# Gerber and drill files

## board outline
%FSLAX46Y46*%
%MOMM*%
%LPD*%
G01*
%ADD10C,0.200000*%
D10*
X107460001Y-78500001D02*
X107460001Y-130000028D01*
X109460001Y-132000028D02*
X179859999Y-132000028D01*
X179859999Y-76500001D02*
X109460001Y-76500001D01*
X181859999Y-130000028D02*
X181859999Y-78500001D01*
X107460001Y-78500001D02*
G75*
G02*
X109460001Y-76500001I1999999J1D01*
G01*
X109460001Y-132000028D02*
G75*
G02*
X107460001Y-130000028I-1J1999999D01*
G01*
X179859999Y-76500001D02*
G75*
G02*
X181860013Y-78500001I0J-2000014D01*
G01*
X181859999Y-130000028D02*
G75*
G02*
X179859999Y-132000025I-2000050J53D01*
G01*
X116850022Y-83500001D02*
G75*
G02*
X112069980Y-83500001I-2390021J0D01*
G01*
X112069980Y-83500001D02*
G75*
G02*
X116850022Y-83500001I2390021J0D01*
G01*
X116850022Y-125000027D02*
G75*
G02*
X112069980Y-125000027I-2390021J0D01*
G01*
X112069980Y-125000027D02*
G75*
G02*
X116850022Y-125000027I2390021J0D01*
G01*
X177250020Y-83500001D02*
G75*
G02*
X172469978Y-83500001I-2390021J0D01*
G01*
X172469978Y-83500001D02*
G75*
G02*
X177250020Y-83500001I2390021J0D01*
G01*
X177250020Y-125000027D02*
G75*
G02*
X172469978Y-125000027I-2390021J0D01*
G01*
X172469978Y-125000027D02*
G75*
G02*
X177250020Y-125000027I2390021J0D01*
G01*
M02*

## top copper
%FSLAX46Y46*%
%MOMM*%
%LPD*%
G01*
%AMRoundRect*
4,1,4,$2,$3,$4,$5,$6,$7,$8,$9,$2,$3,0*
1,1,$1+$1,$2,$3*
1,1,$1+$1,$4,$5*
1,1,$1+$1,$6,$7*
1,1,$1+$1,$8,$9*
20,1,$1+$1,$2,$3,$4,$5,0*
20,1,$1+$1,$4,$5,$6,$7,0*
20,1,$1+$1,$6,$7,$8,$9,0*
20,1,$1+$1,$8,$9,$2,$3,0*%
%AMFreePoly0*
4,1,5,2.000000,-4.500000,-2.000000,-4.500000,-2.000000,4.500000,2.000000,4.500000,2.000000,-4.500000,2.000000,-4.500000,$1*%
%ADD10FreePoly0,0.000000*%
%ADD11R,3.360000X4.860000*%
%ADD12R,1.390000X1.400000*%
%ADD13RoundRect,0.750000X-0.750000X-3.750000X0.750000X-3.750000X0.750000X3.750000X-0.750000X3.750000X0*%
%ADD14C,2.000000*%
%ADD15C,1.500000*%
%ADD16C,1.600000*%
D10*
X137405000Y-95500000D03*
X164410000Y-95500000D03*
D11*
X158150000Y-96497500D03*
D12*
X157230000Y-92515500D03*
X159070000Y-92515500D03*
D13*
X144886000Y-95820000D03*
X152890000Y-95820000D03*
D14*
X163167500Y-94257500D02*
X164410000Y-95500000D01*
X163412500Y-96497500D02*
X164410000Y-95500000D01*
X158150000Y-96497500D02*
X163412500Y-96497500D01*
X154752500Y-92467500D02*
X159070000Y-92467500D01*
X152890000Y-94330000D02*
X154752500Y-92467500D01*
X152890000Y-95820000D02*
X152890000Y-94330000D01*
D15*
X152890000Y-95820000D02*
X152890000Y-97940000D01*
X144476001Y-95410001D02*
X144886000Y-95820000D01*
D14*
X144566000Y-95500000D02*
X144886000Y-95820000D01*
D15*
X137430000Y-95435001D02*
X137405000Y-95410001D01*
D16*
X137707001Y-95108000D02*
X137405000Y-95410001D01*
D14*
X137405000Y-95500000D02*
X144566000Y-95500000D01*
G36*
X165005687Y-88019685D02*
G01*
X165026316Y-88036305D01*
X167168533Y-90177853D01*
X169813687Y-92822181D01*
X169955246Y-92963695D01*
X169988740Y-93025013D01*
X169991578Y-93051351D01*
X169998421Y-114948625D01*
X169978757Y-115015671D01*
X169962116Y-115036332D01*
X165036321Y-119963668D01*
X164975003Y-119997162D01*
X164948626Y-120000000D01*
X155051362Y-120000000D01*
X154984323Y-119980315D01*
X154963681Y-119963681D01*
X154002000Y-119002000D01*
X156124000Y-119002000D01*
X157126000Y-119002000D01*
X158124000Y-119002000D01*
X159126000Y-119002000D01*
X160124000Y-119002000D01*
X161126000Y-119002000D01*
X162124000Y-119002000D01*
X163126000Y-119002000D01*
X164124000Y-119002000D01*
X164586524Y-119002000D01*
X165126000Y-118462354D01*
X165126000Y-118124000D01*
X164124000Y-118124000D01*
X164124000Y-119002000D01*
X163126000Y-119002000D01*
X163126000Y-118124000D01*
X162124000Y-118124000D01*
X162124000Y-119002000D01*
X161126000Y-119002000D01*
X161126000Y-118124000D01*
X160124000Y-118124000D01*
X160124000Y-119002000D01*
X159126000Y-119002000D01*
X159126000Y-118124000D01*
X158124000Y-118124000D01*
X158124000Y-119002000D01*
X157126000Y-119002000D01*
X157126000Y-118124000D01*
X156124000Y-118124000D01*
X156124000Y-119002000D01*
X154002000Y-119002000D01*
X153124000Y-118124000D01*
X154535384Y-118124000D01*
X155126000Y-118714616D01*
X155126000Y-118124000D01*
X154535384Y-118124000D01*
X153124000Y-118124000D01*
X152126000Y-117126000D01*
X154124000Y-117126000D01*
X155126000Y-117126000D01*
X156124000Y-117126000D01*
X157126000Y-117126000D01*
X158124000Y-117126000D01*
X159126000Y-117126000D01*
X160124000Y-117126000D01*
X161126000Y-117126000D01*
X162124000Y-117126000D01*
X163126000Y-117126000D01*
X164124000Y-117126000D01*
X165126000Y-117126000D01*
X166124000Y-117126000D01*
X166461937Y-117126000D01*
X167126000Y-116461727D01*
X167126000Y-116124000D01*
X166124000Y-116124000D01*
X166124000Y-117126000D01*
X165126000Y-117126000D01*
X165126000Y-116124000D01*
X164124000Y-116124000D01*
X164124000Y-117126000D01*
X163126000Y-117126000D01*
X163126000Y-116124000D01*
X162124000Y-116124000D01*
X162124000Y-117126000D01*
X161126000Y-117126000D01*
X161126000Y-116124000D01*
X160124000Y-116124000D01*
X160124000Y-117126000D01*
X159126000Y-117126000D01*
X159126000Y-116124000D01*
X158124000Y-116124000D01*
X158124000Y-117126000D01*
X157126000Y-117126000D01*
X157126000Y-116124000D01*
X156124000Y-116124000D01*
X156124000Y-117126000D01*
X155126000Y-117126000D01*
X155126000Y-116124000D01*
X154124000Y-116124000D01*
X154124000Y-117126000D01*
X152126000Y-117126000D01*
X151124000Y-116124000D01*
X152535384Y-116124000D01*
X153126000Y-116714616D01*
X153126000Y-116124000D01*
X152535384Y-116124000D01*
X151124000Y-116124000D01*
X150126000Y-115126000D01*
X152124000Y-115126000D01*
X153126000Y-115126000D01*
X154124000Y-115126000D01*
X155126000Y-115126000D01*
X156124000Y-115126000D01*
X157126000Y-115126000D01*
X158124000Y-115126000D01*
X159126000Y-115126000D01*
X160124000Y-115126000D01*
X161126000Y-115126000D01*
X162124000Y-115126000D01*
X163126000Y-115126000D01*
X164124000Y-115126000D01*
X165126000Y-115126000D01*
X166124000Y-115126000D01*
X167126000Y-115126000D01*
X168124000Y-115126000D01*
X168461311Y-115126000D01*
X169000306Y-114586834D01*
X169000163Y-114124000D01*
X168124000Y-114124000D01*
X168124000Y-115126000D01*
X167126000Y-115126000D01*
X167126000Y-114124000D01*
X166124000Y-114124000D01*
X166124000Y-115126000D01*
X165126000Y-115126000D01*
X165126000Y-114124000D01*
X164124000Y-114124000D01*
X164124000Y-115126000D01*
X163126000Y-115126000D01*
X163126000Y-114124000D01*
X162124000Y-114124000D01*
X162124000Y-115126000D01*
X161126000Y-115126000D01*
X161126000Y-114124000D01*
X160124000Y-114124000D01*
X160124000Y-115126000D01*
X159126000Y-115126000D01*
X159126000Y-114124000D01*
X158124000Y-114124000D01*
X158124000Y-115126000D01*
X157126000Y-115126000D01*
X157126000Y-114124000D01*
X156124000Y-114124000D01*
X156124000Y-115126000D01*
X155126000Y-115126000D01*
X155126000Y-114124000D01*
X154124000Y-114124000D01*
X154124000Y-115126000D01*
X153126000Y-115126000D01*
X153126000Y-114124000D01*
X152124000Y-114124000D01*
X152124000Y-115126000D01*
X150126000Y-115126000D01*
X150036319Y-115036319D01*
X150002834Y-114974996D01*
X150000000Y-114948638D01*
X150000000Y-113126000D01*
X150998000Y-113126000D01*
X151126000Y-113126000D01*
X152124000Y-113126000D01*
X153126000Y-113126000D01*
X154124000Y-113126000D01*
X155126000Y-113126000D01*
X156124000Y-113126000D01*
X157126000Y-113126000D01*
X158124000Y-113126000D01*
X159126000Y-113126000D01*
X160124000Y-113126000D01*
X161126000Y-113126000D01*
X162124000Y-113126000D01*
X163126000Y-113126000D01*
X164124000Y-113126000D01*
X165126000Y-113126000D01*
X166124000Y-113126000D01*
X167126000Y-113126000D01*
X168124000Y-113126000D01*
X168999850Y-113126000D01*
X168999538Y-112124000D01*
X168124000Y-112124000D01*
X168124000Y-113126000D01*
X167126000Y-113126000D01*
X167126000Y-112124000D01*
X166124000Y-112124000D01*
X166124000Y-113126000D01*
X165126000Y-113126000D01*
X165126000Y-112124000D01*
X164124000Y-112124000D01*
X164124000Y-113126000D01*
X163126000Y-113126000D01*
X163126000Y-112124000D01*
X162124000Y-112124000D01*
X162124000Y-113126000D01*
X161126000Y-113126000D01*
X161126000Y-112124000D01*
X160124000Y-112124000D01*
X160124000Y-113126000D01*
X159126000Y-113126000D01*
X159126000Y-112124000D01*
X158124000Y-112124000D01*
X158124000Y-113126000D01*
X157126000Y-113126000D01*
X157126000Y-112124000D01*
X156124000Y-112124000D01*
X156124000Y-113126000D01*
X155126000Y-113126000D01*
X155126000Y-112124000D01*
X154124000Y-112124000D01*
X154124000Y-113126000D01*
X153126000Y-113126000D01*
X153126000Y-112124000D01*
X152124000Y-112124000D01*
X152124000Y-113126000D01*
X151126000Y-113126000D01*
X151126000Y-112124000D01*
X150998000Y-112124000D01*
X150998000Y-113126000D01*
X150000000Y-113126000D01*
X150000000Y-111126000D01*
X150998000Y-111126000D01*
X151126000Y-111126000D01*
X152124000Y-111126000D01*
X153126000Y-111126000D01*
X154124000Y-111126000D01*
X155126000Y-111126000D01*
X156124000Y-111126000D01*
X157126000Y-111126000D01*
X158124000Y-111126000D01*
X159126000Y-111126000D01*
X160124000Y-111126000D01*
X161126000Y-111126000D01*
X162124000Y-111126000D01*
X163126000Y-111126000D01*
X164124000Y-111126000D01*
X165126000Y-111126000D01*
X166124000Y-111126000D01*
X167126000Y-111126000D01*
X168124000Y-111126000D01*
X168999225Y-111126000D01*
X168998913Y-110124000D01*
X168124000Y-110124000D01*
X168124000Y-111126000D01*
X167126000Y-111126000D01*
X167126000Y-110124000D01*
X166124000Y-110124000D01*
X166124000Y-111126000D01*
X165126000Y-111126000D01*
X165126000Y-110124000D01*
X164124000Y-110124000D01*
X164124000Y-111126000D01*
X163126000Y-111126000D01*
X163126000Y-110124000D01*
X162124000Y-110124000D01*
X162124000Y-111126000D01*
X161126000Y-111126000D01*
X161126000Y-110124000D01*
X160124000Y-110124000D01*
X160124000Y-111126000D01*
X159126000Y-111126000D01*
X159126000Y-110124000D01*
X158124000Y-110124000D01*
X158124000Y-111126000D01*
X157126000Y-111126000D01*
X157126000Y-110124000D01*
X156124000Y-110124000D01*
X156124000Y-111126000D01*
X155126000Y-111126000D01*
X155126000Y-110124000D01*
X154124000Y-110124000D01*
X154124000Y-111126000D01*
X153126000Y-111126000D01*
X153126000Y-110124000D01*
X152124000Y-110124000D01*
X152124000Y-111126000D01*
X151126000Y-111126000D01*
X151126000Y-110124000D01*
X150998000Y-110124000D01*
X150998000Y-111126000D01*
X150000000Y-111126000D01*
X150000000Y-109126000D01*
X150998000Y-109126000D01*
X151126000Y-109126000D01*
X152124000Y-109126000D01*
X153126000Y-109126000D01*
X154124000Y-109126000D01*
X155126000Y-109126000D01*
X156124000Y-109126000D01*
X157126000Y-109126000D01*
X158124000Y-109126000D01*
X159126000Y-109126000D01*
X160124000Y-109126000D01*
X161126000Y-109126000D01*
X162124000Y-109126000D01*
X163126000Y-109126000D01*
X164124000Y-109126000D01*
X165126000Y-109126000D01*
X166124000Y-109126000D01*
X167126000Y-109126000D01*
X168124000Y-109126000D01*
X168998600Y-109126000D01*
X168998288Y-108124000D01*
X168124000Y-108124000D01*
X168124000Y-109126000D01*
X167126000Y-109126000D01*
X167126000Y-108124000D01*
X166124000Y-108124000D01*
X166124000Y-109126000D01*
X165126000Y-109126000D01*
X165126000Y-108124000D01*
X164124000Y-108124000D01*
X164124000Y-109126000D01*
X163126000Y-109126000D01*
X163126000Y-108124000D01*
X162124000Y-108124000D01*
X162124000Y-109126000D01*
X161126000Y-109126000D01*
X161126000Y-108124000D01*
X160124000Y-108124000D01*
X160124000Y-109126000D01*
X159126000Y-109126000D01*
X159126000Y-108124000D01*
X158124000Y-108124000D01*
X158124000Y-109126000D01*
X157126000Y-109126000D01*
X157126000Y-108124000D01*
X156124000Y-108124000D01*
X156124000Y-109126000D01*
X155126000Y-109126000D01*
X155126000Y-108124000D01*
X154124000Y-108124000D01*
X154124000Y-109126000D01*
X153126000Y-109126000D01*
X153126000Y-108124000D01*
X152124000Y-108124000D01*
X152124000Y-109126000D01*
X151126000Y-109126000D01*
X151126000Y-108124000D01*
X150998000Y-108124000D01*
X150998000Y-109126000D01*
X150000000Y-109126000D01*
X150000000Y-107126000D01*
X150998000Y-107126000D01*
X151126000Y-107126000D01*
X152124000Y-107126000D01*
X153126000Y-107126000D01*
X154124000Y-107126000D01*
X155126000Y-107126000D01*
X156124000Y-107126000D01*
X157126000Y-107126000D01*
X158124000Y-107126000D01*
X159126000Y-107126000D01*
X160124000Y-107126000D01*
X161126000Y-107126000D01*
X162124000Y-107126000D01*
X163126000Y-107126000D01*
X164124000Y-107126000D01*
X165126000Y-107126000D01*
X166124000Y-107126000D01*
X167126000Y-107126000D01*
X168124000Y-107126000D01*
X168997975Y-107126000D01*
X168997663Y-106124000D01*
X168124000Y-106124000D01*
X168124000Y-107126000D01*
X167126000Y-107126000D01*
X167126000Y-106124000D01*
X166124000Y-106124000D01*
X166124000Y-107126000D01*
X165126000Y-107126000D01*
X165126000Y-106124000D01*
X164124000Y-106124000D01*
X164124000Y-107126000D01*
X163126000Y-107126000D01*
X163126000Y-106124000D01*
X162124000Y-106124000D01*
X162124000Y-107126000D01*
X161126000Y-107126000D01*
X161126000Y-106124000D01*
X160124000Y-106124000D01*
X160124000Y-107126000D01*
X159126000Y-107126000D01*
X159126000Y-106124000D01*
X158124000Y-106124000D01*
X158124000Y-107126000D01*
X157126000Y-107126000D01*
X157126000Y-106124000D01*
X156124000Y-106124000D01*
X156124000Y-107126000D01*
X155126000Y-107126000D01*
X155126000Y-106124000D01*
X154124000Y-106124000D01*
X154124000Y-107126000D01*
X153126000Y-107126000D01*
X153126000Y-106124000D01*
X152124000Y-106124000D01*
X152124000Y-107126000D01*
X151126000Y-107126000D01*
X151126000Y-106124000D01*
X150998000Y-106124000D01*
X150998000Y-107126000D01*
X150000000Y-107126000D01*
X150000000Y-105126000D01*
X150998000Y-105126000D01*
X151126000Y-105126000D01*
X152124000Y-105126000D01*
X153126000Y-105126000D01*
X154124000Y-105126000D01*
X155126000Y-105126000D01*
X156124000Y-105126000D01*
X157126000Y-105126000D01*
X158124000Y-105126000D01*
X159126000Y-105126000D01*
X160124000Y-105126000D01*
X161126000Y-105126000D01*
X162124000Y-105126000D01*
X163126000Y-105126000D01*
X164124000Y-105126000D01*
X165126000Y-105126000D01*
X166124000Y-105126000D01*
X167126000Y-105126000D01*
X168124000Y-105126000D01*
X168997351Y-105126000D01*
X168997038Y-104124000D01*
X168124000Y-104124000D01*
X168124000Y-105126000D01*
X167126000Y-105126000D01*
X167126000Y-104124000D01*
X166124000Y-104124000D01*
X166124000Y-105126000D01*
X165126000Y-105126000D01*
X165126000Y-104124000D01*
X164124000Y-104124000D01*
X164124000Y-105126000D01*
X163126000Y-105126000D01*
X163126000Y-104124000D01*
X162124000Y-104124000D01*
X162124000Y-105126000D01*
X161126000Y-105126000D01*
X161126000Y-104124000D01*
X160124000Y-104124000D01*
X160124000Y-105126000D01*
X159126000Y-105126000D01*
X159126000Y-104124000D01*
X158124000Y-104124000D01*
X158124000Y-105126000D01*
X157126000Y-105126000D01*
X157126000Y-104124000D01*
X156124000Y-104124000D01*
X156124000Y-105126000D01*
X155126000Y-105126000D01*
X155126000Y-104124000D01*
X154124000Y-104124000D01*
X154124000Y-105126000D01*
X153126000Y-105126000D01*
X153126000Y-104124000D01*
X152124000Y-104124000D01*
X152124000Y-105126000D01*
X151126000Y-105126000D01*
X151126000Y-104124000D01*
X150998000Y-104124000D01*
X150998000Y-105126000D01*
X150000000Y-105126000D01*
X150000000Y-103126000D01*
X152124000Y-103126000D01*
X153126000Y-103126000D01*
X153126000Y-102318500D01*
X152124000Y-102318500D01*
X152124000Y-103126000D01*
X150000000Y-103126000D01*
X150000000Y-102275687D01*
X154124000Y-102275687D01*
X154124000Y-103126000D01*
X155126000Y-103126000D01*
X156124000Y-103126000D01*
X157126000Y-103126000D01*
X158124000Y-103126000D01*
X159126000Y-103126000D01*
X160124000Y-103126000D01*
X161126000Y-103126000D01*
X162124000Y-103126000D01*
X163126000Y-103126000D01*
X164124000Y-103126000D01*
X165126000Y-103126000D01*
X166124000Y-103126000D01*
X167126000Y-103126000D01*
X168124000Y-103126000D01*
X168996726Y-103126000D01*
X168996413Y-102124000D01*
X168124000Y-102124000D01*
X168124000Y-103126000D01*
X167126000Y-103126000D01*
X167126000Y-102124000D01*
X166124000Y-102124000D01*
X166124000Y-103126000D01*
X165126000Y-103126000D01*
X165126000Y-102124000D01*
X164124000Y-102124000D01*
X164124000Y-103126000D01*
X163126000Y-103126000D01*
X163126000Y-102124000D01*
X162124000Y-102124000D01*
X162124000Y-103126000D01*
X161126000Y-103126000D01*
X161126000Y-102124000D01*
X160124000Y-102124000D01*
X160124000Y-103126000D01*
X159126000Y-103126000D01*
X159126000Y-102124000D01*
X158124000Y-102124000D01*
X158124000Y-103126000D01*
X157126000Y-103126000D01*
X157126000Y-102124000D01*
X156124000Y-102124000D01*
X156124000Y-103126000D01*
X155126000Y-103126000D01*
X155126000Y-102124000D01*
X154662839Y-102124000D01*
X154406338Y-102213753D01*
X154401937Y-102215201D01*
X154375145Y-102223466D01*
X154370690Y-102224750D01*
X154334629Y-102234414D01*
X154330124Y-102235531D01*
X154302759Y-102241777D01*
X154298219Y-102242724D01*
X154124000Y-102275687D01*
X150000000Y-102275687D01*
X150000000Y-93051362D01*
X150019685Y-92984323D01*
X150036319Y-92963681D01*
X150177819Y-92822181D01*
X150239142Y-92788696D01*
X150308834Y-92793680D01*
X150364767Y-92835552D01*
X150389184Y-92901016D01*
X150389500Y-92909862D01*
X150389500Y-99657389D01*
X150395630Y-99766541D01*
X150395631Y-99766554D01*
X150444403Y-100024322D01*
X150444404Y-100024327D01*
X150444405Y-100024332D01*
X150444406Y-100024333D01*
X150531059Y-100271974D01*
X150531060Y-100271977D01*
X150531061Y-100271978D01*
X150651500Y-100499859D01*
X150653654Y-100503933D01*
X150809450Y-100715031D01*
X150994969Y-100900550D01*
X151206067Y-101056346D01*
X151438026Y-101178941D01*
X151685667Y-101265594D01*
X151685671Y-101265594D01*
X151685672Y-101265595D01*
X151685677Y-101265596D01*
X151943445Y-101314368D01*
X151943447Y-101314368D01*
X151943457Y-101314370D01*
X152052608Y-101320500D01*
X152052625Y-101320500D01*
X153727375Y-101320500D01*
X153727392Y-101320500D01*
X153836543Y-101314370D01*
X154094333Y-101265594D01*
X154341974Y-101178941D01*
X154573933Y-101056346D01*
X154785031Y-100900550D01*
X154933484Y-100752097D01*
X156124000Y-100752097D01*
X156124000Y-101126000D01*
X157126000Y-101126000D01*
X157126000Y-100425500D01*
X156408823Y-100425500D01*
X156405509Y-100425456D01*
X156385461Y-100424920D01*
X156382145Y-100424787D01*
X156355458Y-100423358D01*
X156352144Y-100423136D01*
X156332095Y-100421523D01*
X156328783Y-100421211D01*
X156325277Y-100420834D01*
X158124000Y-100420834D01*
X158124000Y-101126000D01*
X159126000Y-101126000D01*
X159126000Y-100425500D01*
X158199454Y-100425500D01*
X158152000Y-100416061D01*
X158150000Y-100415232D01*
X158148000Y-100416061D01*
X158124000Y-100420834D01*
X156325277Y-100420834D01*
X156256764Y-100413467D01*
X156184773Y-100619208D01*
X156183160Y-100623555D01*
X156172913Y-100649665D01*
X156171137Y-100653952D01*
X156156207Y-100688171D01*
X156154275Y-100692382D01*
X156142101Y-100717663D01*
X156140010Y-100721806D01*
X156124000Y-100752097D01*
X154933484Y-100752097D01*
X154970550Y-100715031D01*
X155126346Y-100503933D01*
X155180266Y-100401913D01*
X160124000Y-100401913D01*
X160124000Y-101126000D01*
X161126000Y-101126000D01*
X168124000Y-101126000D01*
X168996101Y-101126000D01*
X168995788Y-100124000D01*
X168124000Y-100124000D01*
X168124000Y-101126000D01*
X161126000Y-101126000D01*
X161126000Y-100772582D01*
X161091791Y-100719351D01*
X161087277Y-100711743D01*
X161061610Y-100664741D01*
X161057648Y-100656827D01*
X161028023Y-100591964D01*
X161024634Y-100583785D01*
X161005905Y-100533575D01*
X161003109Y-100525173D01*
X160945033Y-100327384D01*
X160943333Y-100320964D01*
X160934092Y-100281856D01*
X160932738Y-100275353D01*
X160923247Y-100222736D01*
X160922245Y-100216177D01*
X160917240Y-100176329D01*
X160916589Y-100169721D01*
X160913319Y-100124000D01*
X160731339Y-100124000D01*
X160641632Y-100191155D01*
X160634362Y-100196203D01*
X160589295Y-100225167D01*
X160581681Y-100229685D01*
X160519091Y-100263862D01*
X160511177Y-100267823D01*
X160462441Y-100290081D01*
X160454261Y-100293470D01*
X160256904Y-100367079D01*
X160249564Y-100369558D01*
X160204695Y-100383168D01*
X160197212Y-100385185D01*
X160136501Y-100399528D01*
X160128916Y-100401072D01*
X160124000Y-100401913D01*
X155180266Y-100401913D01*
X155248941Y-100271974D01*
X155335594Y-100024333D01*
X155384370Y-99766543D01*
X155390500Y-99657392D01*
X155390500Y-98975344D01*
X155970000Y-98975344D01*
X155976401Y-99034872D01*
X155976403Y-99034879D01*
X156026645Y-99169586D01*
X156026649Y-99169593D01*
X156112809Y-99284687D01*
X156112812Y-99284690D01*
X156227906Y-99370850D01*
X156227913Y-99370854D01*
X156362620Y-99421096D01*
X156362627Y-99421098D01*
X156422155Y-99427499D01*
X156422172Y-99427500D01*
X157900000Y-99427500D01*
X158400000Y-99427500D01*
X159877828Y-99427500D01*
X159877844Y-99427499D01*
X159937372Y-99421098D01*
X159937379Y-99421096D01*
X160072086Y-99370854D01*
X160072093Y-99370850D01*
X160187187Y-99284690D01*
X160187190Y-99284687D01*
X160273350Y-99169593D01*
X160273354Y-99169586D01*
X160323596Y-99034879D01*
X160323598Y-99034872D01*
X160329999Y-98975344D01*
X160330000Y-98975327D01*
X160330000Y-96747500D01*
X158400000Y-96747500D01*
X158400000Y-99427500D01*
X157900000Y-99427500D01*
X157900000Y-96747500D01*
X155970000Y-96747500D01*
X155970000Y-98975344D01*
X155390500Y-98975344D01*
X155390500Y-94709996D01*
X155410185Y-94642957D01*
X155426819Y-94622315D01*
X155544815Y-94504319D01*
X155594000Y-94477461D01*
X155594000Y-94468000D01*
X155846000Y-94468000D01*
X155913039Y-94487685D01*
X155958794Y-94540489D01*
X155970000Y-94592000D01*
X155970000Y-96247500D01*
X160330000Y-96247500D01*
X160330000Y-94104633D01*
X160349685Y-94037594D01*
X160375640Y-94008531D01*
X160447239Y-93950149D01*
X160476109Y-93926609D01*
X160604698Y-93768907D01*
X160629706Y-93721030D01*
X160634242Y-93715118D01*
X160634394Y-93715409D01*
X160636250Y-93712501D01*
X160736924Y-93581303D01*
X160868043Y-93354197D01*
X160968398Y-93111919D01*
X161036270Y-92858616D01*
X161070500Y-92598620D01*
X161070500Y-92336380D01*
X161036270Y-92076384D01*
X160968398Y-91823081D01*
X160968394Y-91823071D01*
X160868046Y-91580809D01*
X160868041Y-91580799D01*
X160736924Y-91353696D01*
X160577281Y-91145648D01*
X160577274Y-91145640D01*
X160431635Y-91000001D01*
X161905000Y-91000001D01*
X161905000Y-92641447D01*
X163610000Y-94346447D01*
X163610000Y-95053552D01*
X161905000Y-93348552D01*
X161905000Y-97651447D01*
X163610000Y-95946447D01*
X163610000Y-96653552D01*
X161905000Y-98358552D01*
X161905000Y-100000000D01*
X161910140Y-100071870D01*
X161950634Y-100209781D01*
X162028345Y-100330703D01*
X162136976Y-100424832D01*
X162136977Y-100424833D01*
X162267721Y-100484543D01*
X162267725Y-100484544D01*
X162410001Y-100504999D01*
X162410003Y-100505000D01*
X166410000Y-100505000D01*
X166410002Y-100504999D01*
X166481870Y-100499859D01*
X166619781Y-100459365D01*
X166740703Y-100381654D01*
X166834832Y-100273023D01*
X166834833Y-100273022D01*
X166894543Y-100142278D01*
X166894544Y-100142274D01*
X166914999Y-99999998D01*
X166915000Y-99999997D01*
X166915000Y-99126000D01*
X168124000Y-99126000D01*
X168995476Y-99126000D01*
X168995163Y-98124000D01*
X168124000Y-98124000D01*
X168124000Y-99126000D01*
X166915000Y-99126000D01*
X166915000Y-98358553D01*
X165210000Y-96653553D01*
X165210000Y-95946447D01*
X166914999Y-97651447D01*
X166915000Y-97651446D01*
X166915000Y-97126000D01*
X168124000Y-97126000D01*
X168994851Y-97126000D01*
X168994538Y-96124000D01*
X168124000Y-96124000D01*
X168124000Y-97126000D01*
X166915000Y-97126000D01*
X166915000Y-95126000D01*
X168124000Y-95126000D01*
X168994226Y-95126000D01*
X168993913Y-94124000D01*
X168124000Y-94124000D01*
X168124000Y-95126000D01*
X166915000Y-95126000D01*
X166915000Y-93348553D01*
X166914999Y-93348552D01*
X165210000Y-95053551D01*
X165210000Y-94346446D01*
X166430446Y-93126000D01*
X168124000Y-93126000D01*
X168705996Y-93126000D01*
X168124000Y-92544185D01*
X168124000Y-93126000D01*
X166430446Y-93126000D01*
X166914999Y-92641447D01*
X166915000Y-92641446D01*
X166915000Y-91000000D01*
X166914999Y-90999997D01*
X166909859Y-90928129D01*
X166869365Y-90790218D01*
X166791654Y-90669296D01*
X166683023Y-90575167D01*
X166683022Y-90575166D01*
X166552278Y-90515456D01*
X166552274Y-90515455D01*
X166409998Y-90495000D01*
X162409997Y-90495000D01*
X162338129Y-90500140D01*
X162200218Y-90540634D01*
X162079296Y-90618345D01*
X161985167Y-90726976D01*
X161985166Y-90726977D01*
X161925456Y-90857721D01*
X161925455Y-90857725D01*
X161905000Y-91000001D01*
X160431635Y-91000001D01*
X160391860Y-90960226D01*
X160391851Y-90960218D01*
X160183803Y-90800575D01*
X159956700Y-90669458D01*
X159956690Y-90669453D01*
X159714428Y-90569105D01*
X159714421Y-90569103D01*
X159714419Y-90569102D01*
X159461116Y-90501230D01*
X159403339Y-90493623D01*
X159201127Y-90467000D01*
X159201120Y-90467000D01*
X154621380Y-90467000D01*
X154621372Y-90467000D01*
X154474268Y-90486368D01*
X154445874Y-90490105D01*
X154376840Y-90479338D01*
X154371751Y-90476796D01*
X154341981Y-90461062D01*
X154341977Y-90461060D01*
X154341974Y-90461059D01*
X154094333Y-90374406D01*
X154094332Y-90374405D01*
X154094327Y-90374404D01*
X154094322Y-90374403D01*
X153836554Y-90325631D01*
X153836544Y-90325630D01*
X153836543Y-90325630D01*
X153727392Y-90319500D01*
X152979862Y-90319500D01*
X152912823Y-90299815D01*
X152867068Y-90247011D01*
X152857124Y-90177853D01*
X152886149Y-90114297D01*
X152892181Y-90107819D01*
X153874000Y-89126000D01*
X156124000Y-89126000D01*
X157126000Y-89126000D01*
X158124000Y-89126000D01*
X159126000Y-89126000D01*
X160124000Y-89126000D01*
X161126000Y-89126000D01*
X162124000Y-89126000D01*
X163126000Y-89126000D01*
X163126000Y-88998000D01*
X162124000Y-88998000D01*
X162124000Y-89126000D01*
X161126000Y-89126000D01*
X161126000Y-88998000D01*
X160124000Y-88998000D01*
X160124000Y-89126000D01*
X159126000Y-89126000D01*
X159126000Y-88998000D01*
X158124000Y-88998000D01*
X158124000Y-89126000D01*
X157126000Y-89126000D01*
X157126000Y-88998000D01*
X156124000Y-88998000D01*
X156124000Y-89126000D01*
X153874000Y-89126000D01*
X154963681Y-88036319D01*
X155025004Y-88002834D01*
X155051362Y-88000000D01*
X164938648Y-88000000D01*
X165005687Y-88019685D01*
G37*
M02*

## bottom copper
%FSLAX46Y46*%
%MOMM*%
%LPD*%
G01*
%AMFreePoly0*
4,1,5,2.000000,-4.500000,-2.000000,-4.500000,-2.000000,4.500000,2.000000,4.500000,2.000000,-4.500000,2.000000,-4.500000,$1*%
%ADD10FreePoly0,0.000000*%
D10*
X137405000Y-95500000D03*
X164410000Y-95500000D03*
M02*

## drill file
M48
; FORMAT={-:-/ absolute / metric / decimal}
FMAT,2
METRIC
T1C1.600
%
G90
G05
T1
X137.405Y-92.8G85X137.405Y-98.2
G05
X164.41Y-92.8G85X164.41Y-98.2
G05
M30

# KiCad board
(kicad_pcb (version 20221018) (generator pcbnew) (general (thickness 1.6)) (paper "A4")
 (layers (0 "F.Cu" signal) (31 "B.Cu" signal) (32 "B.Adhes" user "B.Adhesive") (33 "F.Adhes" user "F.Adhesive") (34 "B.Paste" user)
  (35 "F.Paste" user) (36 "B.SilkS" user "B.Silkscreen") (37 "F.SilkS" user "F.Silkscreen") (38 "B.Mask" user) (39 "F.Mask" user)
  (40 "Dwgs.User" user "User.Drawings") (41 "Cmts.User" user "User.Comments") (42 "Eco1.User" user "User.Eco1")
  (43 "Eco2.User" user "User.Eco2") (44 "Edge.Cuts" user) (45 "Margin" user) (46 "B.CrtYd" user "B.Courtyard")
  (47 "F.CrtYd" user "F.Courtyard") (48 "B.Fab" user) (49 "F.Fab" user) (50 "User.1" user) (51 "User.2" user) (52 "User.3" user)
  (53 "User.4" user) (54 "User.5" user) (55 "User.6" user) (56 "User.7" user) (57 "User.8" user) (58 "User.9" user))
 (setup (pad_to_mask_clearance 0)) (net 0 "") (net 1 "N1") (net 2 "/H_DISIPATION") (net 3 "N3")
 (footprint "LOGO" (layer "F.Cu") (at 160.655 81.915)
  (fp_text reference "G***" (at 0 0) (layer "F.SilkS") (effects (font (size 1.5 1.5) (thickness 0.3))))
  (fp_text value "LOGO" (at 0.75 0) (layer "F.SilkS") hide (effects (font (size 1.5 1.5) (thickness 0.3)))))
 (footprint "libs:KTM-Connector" (layer "F.Cu") (at 144.521999 104.250015)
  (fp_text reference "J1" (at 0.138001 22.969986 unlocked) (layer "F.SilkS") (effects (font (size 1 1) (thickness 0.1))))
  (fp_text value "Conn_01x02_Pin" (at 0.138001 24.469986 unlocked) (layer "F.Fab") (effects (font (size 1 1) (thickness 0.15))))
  (fp_line (start -37.061998 -25.750014) (end -37.061998 25.750013) (stroke (width 0.2) (type solid)) (layer "Edge.Cuts"))
  (fp_line (start -35.061998 27.750013) (end 35.338 27.750013) (stroke (width 0.2) (type solid)) (layer "Edge.Cuts"))
  (fp_line (start 35.338 -27.750014) (end -35.061998 -27.750014) (stroke (width 0.2) (type solid)) (layer "Edge.Cuts"))
  (fp_line (start 37.338 25.750013) (end 37.338 -25.750014) (stroke (width 0.2) (type solid)) (layer "Edge.Cuts"))
  (fp_arc (start -37.061998 -25.750014) (mid -36.476212 -27.164228) (end -35.061998 -27.750014) (stroke (width 0.2) (type solid))
   (layer "Edge.Cuts"))
  (fp_arc (start -35.061998 27.750013) (mid -36.476212 27.164227) (end -37.061998 25.750013) (stroke (width 0.2) (type solid))
   (layer "Edge.Cuts"))
  (fp_arc (start 35.338 -27.750014) (mid 36.752219 -27.164228) (end 37.338 -25.750014) (stroke (width 0.2) (type solid)) (layer "Edge.Cuts"))
  (fp_arc (start 37.338 25.750013) (mid 36.752198 27.16421) (end 35.338 27.750013) (stroke (width 0.2) (type solid)) (layer "Edge.Cuts"))
  (fp_circle (center -30.061998 -20.750014) (end -27.671977 -20.750014) (stroke (width 0.2) (type default)) (fill none) (layer "Edge.Cuts"))
  (fp_circle (center -30.061998 20.750012) (end -27.671977 20.750012) (stroke (width 0.2) (type default)) (fill none) (layer "Edge.Cuts"))
  (fp_circle (center 30.338 -20.750014) (end 32.728021 -20.750014) (stroke (width 0.2) (type default)) (fill none) (layer "Edge.Cuts"))
  (fp_circle (center 30.338 20.750012) (end 32.728021 20.750012) (stroke (width 0.2) (type default)) (fill none) (layer "Edge.Cuts"))
  (pad "1" thru_hole custom (at -7.116999 -8.750015) (size 4 9) (drill oval 1.6 7) (layers "*.Cu" "*.Mask") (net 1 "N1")
   (thermal_bridge_angle 45) (options (clearance outline) (anchor rect)) (primitives))
  (pad "2" thru_hole custom (at 19.888001 -8.750015) (size 4 9) (drill oval 1.6 7) (layers "*.Cu" "*.Mask") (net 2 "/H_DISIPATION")
   (thermal_bridge_angle 45) (options (clearance outline) (anchor rect)) (primitives)))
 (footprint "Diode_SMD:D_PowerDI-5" (layer "F.Cu") (at 158.15 95.3775 90)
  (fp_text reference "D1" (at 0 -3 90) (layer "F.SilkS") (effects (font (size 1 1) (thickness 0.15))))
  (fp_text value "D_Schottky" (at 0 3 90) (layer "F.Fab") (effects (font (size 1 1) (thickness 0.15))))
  (pad "1" smd rect (at -1.12 0 270) (size 4.86 3.36) (layers "F.Cu" "F.Paste" "F.Mask") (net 2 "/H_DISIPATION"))
  (pad "2" smd rect (at 2.862 -0.92 270) (size 1.4 1.39) (layers "F.Cu" "F.Paste" "F.Mask") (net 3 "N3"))
  (pad "2" smd rect (at 2.862 0.92 270) (size 1.4 1.39) (layers "F.Cu" "F.Paste" "F.Mask") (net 3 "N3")))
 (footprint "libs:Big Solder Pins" (layer "F.Cu") (at 148.95 101.92)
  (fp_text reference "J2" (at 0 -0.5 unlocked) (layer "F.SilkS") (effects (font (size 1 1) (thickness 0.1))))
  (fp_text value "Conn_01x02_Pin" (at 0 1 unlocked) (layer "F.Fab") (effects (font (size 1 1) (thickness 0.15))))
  (pad "1" smd roundrect (at -4.064 -6.1) (size 3 9) (layers "F.Cu" "F.Paste" "F.Mask") (roundrect_rratio 0.25) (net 1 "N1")
   (thermal_bridge_angle 45))
  (pad "2" smd roundrect (at 3.94 -6.1) (size 3 9) (layers "F.Cu" "F.Paste" "F.Mask") (roundrect_rratio 0.25) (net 3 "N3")
   (thermal_bridge_angle 45)))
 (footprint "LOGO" (layer "F.Cu") (at 161.29 127)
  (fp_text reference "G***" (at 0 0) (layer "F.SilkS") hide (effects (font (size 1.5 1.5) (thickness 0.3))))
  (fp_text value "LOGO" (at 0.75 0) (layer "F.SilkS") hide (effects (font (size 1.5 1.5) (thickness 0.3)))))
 (segment (start 163.1675 94.2575) (end 164.41 95.5) (width 2) (layer "F.Cu") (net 2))
 (segment (start 163.4125 96.4975) (end 164.41 95.5) (width 2) (layer "F.Cu") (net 2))
 (segment (start 158.15 96.4975) (end 163.4125 96.4975) (width 2) (layer "F.Cu") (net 2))
 (segment (start 154.7525 92.4675) (end 159.07 92.4675) (width 2) (layer "F.Cu") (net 3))
 (segment (start 152.89 94.33) (end 154.7525 92.4675) (width 2) (layer "F.Cu") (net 3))
 (segment (start 152.89 95.82) (end 152.89 94.33) (width 2) (layer "F.Cu") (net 3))
 (segment (start 152.89 95.82) (end 152.89 97.94) (width 1.5) (layer "F.Cu") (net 3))
 (segment (start 144.476001 95.410001) (end 144.886 95.82) (width 1.5) (layer "F.Cu") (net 1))
 (segment (start 144.566 95.5) (end 144.886 95.82) (width 2) (layer "F.Cu") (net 1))
 (segment (start 137.43 95.435001) (end 137.405 95.410001) (width 1.5) (layer "F.Cu") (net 1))
 (segment (start 137.707001 95.108) (end 137.405 95.410001) (width 1.6) (layer "F.Cu") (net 1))
 (segment (start 137.405 95.5) (end 144.566 95.5) (width 2) (layer "F.Cu") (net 1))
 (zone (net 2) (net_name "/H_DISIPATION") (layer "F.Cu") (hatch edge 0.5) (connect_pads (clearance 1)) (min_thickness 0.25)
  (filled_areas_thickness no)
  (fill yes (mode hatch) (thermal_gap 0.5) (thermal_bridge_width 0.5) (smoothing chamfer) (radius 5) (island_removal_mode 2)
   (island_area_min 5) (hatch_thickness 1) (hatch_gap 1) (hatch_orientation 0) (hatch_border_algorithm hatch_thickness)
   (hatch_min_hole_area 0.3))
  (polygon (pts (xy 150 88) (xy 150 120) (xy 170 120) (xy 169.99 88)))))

